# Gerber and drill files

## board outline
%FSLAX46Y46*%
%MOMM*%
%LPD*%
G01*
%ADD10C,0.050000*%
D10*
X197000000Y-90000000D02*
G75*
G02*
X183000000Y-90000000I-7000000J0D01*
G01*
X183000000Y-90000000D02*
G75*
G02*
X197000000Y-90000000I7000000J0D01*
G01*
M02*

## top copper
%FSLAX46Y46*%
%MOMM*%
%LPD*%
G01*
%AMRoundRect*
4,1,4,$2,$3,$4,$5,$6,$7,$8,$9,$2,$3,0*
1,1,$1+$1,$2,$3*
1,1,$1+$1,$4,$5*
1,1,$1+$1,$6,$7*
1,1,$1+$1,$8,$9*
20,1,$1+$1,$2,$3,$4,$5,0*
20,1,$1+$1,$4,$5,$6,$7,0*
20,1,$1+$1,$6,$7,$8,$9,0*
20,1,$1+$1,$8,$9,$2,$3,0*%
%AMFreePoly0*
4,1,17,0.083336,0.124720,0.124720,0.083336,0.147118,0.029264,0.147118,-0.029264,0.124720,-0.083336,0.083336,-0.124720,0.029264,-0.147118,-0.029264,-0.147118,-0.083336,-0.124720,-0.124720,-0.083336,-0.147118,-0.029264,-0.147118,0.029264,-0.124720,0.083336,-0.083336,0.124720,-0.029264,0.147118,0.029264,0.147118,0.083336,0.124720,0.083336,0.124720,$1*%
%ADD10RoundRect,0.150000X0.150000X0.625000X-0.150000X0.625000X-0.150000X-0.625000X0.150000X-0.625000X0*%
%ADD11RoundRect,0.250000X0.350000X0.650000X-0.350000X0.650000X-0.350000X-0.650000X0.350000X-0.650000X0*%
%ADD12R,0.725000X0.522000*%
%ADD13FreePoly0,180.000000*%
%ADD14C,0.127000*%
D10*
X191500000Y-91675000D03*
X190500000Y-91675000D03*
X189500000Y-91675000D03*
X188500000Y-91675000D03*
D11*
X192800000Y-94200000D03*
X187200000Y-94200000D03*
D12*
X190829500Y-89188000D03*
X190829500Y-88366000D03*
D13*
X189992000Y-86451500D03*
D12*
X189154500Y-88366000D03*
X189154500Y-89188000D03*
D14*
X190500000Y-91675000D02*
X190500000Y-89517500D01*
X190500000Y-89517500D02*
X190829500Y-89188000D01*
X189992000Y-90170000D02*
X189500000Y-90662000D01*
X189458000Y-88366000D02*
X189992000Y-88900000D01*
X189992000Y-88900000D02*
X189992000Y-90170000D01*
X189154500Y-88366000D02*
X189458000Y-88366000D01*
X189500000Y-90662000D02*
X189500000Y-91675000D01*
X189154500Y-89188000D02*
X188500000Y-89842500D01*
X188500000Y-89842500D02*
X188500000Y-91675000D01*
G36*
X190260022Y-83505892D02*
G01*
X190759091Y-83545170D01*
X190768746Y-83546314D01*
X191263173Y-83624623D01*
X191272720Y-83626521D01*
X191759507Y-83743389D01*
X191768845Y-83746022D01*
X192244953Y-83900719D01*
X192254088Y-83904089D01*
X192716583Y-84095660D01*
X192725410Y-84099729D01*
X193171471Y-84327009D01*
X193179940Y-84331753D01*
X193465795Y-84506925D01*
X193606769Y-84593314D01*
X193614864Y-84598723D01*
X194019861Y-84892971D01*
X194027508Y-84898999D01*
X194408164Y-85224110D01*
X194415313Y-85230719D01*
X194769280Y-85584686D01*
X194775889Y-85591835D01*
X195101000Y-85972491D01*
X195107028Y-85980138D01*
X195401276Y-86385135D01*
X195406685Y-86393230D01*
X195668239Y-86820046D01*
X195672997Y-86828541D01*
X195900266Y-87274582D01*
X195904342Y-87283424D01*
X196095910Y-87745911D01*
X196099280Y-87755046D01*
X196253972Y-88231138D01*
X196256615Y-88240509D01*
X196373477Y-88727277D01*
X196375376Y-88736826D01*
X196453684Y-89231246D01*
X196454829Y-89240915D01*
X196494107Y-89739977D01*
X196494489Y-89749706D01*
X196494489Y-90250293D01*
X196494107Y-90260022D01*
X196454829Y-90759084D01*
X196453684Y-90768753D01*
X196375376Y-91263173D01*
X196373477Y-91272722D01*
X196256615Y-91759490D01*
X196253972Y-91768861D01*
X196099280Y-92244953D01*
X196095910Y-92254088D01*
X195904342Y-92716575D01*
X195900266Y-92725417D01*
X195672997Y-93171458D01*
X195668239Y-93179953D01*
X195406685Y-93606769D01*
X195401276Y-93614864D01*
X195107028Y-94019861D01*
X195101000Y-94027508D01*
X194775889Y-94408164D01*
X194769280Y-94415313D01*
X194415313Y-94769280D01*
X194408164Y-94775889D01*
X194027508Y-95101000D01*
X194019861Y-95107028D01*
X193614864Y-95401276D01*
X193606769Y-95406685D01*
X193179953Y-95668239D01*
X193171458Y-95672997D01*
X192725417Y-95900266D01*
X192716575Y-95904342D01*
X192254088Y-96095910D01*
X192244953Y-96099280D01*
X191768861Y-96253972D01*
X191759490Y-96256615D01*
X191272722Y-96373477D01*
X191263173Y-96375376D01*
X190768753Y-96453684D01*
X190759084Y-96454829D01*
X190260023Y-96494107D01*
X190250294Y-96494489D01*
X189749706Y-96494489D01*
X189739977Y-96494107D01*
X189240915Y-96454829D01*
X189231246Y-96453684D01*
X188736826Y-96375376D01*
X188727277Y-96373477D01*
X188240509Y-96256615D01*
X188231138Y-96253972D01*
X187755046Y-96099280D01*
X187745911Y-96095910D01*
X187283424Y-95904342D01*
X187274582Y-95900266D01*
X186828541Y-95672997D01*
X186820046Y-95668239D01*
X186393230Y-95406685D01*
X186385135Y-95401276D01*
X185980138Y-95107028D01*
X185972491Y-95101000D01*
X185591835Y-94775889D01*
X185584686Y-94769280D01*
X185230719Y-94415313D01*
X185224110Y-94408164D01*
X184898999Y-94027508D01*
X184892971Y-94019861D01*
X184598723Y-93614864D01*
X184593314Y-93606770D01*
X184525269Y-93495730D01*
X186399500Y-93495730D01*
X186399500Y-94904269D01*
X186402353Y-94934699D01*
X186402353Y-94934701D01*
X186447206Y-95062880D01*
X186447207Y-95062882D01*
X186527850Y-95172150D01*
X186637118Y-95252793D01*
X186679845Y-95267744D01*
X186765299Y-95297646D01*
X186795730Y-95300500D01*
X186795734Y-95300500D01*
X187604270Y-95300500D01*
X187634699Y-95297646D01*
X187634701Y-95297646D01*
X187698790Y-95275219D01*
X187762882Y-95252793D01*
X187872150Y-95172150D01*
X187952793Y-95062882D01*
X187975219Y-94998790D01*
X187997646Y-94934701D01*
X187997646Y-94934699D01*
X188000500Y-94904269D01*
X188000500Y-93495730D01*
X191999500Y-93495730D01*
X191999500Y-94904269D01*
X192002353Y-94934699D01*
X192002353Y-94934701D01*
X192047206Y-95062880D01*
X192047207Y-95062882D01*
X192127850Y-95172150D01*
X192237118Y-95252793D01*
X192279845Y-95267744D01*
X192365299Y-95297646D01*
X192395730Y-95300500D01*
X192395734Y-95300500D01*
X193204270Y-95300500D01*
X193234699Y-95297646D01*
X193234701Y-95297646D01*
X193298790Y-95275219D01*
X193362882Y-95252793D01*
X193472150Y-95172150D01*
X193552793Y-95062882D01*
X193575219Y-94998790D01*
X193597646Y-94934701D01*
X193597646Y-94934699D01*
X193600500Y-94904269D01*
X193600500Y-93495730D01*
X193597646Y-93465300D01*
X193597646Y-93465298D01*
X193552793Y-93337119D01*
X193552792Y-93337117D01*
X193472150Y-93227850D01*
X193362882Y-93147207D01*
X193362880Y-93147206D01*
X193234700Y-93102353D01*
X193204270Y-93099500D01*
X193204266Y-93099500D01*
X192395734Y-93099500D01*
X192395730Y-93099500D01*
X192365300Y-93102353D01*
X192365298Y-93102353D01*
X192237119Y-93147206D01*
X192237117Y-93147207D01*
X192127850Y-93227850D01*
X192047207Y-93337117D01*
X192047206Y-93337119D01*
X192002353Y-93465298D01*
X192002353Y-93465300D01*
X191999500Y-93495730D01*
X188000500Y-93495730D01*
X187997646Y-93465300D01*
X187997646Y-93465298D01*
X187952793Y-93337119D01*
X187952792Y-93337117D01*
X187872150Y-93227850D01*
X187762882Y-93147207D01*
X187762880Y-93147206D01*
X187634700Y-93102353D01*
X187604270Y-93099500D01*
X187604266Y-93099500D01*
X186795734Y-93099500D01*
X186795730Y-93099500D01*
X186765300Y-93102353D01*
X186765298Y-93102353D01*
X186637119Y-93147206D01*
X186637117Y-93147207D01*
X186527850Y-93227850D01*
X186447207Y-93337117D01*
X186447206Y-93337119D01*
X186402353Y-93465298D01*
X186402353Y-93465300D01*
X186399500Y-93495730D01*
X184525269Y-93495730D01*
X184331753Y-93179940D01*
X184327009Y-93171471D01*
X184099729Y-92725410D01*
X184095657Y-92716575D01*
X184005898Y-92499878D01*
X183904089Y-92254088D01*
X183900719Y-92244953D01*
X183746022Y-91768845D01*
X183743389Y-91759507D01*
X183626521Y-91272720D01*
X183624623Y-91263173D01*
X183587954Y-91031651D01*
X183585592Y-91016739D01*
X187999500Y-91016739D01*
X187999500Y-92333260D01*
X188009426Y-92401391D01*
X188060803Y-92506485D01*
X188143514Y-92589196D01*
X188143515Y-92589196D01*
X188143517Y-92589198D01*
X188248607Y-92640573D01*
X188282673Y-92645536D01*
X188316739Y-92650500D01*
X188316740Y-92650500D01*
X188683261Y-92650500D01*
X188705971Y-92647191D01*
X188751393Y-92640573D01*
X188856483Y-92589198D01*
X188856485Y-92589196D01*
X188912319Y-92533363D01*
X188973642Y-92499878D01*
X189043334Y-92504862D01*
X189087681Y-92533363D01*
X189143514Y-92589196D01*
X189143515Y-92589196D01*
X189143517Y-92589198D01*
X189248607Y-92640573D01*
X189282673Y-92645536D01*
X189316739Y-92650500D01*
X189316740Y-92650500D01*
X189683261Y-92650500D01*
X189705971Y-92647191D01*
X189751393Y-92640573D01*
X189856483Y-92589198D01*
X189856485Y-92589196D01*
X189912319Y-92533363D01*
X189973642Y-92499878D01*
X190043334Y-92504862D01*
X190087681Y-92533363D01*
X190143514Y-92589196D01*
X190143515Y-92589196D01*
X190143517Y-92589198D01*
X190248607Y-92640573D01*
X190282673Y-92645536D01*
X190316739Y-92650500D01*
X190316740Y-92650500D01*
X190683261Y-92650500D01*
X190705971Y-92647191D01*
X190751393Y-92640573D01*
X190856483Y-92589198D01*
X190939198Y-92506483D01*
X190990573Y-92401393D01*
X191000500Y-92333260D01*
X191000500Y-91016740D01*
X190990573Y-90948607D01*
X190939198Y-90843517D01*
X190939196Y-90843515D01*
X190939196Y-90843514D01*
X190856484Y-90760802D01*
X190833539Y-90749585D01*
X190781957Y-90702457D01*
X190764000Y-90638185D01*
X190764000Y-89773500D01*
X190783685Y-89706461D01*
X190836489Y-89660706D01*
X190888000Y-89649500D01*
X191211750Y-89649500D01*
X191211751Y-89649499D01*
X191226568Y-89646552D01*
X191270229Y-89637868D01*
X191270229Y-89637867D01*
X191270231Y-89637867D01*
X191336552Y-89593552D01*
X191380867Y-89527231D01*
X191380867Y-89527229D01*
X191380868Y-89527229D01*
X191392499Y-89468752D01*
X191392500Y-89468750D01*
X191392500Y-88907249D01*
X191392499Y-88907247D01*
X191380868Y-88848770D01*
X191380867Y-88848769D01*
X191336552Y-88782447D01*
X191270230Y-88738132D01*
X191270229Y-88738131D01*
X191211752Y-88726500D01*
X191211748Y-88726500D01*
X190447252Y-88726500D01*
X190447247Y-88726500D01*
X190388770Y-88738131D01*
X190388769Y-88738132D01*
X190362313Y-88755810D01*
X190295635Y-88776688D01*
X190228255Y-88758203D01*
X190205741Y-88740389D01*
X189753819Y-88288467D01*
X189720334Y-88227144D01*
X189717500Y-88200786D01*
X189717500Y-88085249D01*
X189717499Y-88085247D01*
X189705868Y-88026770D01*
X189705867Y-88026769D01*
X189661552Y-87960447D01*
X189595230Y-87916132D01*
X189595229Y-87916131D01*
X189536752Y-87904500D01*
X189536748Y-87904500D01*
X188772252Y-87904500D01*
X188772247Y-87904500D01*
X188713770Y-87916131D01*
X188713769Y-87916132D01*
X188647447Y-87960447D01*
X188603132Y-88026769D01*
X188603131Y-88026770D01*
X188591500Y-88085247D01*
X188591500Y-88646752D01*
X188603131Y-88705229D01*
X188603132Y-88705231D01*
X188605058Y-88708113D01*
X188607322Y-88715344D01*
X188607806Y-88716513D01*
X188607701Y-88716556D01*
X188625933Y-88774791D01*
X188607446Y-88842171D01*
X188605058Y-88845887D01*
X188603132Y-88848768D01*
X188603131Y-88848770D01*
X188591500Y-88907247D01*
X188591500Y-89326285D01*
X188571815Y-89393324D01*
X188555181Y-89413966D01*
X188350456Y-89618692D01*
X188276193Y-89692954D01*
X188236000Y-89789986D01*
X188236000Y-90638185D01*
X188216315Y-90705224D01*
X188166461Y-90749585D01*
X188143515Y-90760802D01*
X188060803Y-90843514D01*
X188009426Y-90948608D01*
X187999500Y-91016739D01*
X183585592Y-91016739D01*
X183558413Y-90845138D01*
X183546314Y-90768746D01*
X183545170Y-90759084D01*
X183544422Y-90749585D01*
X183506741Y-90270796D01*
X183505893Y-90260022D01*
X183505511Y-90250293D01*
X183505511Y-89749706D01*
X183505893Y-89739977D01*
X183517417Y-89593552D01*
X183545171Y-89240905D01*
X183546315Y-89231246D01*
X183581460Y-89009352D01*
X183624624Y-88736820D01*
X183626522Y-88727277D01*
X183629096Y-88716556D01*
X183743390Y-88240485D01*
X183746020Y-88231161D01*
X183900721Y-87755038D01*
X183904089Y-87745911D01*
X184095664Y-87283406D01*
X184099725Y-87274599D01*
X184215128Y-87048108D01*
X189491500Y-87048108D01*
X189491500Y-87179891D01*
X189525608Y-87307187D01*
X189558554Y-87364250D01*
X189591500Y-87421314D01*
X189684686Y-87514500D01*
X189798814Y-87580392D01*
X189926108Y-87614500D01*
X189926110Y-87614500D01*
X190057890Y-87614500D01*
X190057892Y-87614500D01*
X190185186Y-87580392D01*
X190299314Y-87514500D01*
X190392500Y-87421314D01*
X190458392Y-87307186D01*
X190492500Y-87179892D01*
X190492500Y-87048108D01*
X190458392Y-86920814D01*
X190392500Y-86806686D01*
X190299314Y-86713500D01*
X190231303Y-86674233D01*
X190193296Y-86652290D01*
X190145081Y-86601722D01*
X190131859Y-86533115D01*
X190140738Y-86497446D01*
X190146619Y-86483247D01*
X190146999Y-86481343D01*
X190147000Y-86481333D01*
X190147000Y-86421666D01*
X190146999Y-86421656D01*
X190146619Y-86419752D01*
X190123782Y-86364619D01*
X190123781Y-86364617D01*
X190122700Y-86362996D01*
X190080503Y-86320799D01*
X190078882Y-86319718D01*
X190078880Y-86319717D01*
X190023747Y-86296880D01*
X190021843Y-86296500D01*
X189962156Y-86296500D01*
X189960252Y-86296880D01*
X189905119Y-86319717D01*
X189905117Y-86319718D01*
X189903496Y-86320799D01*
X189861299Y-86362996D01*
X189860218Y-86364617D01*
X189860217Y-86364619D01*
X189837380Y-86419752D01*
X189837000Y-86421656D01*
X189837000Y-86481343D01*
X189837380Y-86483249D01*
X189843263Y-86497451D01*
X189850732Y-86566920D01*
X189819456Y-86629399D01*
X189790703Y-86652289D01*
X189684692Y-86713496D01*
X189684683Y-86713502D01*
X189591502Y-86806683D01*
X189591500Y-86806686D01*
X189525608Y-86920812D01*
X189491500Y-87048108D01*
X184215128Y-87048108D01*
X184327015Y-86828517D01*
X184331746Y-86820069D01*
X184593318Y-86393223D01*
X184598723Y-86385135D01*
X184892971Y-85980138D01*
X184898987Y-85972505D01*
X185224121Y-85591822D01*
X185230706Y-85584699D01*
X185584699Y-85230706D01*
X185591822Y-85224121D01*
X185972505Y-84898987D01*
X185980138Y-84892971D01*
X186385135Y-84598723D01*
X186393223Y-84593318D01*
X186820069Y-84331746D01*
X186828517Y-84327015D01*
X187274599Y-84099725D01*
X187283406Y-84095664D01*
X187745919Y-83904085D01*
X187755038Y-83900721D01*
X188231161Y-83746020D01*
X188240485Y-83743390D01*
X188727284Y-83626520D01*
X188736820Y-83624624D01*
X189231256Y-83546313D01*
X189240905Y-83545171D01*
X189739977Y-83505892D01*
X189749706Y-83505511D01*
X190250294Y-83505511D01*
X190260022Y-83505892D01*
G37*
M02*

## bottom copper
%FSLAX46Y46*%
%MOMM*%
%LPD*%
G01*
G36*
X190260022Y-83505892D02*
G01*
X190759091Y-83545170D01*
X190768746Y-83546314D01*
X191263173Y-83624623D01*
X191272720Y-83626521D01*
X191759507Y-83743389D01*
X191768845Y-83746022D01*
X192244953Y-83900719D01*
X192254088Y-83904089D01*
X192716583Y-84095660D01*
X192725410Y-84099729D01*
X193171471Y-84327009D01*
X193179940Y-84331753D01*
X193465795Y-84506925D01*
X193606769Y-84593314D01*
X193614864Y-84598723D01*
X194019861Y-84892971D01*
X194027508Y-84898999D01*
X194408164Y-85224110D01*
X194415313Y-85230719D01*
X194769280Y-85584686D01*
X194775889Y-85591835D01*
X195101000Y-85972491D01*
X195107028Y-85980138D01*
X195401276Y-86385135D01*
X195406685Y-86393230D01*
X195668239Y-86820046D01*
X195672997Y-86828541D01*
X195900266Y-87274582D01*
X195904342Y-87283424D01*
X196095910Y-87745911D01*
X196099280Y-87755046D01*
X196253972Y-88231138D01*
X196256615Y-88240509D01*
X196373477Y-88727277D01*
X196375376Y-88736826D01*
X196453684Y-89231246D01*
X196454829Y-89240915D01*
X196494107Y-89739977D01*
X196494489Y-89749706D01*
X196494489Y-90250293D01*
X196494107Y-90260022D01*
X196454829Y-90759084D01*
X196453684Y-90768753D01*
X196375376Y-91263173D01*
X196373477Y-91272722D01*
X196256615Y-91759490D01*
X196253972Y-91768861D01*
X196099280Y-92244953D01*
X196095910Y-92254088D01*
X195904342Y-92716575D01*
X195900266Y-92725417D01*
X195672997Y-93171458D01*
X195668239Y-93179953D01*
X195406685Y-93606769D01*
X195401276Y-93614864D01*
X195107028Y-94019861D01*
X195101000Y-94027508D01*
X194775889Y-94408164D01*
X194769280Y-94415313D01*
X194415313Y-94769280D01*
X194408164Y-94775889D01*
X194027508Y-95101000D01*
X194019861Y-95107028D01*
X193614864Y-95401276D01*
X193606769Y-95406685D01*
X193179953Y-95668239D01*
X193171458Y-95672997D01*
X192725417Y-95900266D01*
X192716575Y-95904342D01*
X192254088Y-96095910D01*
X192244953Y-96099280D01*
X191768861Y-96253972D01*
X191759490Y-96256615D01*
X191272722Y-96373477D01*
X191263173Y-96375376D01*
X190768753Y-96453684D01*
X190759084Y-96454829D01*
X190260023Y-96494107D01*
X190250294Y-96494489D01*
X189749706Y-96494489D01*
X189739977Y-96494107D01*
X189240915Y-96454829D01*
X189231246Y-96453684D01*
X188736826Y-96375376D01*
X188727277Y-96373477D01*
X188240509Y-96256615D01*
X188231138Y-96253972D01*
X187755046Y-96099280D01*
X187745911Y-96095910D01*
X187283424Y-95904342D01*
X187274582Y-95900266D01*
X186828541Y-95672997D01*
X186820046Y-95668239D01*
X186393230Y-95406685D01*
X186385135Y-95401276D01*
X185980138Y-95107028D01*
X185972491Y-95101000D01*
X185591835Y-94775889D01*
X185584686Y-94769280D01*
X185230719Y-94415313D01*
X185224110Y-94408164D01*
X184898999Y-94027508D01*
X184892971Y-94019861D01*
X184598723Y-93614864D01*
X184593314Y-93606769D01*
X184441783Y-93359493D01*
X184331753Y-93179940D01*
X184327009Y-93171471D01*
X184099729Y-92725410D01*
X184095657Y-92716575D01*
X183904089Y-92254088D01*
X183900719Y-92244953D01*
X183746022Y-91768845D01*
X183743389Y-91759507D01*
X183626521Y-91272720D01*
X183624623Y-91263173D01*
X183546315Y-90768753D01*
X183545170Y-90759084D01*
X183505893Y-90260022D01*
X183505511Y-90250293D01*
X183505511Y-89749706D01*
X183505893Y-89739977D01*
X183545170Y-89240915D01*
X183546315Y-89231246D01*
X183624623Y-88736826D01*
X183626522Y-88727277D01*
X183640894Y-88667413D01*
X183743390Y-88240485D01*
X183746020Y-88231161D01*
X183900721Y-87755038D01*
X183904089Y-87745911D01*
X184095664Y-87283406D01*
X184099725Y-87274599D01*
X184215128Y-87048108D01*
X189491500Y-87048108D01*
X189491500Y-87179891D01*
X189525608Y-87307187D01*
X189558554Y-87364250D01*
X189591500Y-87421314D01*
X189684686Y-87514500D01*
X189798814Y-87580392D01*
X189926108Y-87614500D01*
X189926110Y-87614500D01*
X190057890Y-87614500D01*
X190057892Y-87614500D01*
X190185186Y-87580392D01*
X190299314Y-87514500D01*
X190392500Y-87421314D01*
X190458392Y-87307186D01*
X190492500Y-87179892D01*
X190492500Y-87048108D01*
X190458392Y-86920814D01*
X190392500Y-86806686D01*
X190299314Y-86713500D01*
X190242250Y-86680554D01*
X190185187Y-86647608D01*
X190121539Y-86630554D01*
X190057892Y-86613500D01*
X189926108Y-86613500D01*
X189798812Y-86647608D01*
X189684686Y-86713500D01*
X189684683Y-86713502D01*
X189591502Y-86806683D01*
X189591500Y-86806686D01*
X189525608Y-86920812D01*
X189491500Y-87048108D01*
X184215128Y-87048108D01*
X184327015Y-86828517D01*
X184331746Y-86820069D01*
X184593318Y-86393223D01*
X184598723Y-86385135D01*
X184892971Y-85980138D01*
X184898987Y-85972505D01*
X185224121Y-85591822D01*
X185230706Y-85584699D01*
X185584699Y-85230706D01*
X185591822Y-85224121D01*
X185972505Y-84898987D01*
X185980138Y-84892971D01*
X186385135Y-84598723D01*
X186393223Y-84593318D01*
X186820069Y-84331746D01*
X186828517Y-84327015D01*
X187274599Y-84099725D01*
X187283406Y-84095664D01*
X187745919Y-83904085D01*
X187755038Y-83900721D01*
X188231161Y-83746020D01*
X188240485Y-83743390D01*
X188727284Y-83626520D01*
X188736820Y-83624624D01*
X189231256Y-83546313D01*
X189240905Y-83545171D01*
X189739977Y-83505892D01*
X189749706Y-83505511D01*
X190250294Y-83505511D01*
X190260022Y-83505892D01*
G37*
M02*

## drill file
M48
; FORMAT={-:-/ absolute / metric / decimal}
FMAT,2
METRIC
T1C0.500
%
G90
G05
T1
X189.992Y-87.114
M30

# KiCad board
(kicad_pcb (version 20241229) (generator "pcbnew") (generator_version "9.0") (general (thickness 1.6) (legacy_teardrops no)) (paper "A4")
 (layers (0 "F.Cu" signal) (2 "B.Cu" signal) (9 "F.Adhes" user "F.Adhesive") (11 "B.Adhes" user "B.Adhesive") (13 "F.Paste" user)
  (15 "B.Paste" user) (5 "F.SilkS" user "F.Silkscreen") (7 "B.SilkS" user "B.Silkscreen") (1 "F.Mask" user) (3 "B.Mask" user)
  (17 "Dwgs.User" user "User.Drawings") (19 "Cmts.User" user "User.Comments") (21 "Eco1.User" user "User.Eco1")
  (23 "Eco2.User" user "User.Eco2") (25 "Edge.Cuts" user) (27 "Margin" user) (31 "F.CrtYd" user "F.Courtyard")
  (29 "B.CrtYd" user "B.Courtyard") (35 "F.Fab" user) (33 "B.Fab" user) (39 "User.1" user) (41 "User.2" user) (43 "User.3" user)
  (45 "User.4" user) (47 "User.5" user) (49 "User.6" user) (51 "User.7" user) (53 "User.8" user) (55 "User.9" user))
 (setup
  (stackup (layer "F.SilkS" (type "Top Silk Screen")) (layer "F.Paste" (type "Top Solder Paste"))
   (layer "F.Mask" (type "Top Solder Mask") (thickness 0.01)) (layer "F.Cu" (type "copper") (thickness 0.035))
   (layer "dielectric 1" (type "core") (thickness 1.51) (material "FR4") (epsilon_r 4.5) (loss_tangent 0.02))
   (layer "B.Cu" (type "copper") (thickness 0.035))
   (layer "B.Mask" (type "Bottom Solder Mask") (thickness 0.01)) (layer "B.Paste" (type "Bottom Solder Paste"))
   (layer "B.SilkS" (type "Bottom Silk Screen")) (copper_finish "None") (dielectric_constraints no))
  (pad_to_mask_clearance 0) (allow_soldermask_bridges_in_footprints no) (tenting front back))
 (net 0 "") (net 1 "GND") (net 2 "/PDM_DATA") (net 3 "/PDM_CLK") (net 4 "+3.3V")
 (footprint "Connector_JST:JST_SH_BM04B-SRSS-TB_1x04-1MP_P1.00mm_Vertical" (layer "F.Cu") (at 190 93 180)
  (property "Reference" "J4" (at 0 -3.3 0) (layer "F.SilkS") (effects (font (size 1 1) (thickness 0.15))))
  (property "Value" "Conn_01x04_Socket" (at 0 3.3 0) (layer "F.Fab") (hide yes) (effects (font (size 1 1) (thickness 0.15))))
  (pad "1" smd roundrect (at -1.5 1.325 180) (size 0.6 1.55) (layers "F.Cu" "F.Mask" "F.Paste") (roundrect_rratio 0.25) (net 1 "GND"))
  (pad "2" smd roundrect (at -0.5 1.325 180) (size 0.6 1.55) (layers "F.Cu" "F.Mask" "F.Paste") (roundrect_rratio 0.25) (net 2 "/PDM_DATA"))
  (pad "3" smd roundrect (at 0.5 1.325 180) (size 0.6 1.55) (layers "F.Cu" "F.Mask" "F.Paste") (roundrect_rratio 0.25) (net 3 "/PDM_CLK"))
  (pad "4" smd roundrect (at 1.5 1.325 180) (size 0.6 1.55) (layers "F.Cu" "F.Mask" "F.Paste") (roundrect_rratio 0.25) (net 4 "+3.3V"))
  (pad "MP" smd roundrect (at -2.8 -1.2 180) (size 1.2 1.8) (layers "F.Cu" "F.Mask" "F.Paste") (roundrect_rratio 0.208333))
  (pad "MP" smd roundrect (at 2.8 -1.2 180) (size 1.2 1.8) (layers "F.Cu" "F.Mask" "F.Paste") (roundrect_rratio 0.208333)))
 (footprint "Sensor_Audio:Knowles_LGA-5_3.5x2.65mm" (layer "F.Cu") (at 189.992 87.884 180)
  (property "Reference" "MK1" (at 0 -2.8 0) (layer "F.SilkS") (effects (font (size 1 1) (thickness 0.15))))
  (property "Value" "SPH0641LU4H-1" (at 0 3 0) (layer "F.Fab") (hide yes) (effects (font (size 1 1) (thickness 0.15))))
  (pad "" np_thru_hole circle (at 0 0.77 180) (size 0.5 0.5) (drill 0.5) (layers "*.Cu" "*.Mask"))
  (pad "1" smd rect (at -0.8375 -1.304 180) (size 0.725 0.522) (layers "F.Cu" "F.Mask" "F.Paste") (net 2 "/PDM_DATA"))
  (pad "2" smd rect (at -0.8375 -0.482 180) (size 0.725 0.522) (layers "F.Cu" "F.Mask" "F.Paste") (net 1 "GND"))
  (pad "3" smd custom (at 0 1.4325 180) (size 0.3 0.3) (layers "F.Cu" "F.Mask") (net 1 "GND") (zone_connect 0)
   (options (clearance outline) (anchor circle)) (primitives))
  (pad "4" smd rect (at 0.8375 -0.482 180) (size 0.725 0.522) (layers "F.Cu" "F.Mask" "F.Paste") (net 3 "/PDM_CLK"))
  (pad "5" smd rect (at 0.8375 -1.304 180) (size 0.725 0.522) (layers "F.Cu" "F.Mask" "F.Paste") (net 4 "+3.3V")))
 (gr_circle (center 190 90) (end 197 90) (stroke (width 0.05) (type default)) (fill no) (layer "Edge.Cuts"))
 (segment (start 190.5 91.675) (end 190.5 89.5175) (width 0.127) (layer "F.Cu") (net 2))
 (segment (start 190.5 89.5175) (end 190.8295 89.188) (width 0.127) (layer "F.Cu") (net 2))
 (segment (start 189.992 90.17) (end 189.5 90.662) (width 0.127) (layer "F.Cu") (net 3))
 (segment (start 189.458 88.366) (end 189.992 88.9) (width 0.127) (layer "F.Cu") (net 3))
 (segment (start 189.992 88.9) (end 189.992 90.17) (width 0.127) (layer "F.Cu") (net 3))
 (segment (start 189.1545 88.366) (end 189.458 88.366) (width 0.127) (layer "F.Cu") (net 3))
 (segment (start 189.5 90.662) (end 189.5 91.675) (width 0.127) (layer "F.Cu") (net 3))
 (segment (start 189.1545 89.188) (end 188.5 89.8425) (width 0.127) (layer "F.Cu") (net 4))
 (segment (start 188.5 89.8425) (end 188.5 91.675) (width 0.127) (layer "F.Cu") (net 4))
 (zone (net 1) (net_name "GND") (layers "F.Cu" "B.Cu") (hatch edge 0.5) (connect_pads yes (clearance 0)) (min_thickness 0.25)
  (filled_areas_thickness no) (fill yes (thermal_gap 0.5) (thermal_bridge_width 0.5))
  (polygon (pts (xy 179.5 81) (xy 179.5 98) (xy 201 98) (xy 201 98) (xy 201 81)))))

